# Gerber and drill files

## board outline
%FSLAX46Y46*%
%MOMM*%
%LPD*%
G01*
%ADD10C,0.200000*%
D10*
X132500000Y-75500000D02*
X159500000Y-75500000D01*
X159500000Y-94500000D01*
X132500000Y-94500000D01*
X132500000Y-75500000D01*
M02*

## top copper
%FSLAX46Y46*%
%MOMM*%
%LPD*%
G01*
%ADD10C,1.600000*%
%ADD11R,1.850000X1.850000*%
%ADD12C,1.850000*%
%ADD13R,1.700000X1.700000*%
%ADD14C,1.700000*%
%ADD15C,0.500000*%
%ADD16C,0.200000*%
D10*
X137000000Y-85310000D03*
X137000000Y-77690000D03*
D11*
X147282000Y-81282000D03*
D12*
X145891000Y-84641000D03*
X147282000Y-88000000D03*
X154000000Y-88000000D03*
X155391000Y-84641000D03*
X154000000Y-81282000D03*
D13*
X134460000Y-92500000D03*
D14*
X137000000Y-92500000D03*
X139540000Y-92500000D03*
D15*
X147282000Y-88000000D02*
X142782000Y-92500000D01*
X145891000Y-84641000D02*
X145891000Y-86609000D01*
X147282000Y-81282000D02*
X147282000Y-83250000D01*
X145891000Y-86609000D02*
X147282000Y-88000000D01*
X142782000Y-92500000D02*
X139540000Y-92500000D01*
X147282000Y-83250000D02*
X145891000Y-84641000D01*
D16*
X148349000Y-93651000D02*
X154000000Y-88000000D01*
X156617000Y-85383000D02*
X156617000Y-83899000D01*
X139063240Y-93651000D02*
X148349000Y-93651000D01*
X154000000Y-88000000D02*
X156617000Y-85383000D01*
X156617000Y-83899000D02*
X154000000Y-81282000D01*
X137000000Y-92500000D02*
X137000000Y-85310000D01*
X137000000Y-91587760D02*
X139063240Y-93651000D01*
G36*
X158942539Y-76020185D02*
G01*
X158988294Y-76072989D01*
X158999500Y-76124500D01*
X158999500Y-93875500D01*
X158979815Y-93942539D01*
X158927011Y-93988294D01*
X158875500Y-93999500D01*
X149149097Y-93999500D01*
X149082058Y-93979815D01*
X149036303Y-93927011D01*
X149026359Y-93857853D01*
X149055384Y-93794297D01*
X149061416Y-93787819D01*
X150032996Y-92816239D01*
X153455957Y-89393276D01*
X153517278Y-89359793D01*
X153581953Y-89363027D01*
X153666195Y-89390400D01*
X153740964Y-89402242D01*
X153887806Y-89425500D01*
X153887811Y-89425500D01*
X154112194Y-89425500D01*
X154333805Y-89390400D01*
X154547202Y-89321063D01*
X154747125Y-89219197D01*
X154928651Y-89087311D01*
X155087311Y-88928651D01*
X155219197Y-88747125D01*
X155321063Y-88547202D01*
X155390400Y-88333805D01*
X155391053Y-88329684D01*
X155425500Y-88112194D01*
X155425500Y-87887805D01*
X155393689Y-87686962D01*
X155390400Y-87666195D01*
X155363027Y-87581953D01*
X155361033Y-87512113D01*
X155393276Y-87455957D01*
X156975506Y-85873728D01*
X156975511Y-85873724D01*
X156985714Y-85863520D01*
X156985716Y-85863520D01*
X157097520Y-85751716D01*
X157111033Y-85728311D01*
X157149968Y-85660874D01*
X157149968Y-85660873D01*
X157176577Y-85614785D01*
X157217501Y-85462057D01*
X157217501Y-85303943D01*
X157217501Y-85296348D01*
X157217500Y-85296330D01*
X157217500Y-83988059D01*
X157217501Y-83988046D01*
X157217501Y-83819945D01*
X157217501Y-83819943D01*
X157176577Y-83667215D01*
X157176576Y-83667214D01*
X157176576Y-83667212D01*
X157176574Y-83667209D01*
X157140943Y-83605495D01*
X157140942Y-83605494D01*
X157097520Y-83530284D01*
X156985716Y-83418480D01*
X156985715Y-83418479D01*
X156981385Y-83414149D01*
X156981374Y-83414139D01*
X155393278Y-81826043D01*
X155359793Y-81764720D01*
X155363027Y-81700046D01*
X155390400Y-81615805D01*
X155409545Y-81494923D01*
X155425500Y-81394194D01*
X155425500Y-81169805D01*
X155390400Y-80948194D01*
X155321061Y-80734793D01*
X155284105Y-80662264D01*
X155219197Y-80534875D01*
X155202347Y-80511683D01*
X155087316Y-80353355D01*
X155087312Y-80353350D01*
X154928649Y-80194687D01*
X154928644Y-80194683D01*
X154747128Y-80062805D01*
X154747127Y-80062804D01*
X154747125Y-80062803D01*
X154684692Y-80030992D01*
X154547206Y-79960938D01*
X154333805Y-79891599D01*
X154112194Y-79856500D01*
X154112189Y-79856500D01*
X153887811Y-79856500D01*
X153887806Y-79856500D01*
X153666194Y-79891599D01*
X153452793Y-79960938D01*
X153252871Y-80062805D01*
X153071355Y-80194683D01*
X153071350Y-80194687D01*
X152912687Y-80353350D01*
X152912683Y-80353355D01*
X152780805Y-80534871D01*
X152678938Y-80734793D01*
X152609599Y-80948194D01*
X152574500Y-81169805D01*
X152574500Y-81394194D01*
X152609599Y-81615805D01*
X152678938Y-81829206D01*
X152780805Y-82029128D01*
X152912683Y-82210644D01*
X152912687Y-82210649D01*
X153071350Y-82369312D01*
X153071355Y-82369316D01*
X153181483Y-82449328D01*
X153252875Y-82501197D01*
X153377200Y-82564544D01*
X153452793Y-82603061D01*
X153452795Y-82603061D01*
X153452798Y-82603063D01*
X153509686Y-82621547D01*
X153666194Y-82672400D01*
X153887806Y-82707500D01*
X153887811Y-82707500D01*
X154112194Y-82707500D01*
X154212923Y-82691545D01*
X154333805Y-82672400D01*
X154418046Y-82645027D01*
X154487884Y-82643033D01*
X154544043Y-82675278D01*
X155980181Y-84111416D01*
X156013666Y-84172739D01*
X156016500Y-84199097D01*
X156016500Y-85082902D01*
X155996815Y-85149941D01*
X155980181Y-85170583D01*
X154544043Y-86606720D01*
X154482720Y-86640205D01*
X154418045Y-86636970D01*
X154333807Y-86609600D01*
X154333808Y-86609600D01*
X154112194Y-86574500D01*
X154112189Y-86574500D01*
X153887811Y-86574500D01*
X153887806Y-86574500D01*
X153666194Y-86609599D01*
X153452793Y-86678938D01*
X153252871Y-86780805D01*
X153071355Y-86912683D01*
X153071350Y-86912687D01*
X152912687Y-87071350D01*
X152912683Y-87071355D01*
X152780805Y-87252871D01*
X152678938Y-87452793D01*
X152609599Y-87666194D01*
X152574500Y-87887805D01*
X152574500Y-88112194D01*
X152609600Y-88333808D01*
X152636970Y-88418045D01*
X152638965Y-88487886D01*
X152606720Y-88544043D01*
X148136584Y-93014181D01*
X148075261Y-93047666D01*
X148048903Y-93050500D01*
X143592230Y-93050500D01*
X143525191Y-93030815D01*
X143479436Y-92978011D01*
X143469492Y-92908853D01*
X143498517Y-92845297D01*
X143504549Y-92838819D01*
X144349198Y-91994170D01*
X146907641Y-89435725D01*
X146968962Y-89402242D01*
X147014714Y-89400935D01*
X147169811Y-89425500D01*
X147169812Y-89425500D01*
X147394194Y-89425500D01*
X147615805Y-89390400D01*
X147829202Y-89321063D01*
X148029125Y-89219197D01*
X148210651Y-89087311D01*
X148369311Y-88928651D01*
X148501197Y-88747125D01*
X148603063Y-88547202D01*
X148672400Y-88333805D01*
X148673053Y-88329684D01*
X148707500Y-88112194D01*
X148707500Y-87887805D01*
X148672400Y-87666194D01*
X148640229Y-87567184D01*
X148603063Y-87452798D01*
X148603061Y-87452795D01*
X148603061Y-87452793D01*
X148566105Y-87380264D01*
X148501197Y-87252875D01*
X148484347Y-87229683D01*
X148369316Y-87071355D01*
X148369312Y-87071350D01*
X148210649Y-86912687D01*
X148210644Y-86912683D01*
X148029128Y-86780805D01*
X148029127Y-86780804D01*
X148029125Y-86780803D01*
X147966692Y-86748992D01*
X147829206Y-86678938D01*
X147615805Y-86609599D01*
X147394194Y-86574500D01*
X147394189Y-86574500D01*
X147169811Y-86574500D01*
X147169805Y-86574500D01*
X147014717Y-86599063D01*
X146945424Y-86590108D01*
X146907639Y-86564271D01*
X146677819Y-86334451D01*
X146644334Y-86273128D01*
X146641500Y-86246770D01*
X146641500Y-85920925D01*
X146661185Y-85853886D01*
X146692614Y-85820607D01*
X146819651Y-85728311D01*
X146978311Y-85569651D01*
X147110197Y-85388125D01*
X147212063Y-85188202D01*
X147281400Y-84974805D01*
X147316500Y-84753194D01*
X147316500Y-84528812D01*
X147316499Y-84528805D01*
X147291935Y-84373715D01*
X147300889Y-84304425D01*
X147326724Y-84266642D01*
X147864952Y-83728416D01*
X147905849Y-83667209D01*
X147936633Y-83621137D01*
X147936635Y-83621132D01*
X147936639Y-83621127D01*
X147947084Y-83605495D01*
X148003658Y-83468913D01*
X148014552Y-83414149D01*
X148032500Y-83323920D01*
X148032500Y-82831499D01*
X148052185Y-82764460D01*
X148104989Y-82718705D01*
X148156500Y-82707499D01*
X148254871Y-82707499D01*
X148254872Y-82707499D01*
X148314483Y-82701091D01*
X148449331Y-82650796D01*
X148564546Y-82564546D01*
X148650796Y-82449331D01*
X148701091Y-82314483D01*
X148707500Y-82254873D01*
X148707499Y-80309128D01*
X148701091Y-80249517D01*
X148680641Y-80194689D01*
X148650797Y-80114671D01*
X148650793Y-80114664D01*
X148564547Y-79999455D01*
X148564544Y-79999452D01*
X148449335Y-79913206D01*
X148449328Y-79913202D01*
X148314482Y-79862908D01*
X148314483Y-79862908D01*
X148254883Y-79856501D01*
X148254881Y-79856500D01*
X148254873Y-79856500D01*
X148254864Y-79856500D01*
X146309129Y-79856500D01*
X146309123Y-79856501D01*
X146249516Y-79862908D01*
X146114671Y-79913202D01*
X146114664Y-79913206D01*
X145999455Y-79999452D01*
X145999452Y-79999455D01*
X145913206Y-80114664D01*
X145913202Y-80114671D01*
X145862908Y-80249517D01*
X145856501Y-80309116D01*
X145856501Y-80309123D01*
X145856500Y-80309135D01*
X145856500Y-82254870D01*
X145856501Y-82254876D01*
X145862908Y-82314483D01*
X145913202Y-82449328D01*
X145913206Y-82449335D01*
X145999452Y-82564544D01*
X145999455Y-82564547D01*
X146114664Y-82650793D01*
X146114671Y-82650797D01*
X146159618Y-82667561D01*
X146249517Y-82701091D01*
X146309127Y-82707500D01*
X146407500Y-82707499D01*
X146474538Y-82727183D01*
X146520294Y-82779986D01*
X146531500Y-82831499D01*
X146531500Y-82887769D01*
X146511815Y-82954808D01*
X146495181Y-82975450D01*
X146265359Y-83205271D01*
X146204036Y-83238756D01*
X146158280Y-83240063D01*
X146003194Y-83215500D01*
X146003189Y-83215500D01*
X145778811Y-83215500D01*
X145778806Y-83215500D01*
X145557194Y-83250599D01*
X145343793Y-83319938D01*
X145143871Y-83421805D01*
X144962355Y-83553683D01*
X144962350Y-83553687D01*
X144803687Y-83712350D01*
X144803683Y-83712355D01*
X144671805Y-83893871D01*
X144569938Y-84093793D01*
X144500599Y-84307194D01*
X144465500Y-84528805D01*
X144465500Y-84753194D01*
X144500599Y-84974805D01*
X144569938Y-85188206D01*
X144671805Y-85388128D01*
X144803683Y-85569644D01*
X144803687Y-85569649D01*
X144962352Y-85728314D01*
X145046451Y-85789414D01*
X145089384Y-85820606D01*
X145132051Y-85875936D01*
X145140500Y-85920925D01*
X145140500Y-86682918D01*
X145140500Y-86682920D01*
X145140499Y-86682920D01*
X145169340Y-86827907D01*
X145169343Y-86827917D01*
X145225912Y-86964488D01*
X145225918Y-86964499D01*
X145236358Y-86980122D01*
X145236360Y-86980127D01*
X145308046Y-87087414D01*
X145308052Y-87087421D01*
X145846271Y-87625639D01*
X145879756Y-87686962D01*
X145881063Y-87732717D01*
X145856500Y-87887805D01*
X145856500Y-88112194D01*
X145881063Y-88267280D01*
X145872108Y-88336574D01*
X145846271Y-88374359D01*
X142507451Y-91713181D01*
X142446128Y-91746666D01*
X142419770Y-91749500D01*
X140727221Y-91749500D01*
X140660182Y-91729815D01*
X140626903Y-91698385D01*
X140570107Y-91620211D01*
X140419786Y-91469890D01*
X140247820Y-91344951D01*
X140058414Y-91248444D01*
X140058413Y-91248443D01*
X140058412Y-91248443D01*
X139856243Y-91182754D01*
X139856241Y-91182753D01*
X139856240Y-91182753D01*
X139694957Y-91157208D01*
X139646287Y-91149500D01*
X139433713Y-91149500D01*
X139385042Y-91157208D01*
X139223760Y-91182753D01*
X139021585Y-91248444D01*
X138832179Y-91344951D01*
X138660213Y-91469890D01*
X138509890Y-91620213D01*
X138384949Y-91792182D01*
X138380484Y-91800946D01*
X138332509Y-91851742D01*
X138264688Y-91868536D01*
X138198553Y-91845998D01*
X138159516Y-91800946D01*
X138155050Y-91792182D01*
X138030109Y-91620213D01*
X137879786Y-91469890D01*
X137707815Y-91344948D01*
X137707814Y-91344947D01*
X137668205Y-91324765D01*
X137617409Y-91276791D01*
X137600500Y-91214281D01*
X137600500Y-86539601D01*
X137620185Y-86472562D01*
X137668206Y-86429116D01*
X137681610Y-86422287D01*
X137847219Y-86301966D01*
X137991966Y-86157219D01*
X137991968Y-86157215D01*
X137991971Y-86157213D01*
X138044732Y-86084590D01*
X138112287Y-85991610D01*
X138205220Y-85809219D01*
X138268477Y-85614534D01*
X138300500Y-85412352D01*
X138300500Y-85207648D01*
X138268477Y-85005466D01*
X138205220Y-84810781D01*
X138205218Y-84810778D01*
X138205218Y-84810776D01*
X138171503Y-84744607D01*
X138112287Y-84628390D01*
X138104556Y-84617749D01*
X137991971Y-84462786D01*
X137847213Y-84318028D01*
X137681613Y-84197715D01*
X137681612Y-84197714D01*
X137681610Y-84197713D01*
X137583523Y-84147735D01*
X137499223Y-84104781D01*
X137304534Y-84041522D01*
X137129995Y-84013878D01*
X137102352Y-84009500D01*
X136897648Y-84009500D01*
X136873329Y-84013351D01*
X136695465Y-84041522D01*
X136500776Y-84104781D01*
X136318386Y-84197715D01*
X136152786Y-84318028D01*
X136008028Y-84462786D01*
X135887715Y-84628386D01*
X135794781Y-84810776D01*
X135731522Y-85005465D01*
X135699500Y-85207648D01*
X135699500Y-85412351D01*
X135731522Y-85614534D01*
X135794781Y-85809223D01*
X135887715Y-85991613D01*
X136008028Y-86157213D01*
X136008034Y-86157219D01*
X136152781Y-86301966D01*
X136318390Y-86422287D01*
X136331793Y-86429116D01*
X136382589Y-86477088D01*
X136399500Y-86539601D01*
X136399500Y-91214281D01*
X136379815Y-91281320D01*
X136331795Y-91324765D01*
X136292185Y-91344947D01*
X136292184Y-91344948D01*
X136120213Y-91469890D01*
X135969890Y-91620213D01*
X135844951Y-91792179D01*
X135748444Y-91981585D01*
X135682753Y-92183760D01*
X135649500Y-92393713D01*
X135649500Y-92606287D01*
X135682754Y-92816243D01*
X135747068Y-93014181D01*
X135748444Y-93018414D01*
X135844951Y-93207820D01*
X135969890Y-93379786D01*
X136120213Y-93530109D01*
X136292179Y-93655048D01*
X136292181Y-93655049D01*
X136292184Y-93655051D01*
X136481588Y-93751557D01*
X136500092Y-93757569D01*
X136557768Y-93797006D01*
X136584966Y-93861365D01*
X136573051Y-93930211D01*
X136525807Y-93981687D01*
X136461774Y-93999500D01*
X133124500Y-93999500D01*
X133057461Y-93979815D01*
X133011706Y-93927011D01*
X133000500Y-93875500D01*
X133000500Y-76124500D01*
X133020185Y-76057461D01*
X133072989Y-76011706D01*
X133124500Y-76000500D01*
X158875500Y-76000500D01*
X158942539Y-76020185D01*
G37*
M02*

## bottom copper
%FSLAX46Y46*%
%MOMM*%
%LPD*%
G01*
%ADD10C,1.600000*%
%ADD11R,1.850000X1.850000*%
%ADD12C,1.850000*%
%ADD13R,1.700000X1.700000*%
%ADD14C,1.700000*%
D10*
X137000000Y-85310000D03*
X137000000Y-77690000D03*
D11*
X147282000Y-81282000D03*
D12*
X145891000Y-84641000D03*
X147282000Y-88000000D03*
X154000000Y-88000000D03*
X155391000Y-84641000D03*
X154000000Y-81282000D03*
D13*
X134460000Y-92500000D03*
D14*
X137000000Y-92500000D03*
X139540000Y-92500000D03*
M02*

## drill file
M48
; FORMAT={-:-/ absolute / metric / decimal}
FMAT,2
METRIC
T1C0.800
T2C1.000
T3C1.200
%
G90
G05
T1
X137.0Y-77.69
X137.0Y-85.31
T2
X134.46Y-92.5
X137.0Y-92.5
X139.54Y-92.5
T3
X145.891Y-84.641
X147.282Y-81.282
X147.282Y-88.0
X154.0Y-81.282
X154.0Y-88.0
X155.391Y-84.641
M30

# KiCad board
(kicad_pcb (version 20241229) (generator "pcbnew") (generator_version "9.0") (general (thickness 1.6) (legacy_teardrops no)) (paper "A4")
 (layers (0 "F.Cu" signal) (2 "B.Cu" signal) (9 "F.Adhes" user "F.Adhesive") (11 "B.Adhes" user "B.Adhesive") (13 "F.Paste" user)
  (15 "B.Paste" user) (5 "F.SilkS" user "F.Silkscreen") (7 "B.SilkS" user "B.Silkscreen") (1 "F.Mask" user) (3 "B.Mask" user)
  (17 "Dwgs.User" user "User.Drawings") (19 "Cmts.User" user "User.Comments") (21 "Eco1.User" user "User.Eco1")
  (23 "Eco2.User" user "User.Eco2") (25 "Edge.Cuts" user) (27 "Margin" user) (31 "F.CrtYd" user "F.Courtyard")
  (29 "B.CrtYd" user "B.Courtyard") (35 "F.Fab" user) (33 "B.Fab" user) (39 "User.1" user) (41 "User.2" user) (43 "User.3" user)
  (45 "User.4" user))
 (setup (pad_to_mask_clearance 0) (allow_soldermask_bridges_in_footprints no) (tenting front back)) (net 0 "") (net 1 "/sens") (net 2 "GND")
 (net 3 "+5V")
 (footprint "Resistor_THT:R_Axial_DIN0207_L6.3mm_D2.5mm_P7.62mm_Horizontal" (layer "F.Cu") (at 137 85.31 90)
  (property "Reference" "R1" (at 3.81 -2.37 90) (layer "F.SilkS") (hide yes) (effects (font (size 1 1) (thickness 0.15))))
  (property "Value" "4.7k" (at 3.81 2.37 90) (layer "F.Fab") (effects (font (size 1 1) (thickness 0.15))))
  (pad "1" thru_hole circle (at 0 0 90) (size 1.6 1.6) (drill 0.8) (layers "*.Cu" "*.Mask") (remove_unused_layers no) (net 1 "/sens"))
  (pad "2" thru_hole circle (at 7.62 0 90) (size 1.6 1.6) (drill 0.8) (layers "*.Cu" "*.Mask") (remove_unused_layers no) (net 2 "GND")))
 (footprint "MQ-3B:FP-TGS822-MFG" (layer "F.Cu") (at 150.641 84.641)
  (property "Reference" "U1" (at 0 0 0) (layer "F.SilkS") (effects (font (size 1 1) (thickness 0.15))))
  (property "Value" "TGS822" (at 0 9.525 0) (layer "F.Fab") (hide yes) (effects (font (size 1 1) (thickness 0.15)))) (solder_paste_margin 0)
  (pad "1" thru_hole rect (at -3.359 -3.359) (size 1.85 1.85) (drill 1.2) (layers "*.Cu" "*.Mask") (remove_unused_layers no) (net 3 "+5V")
   (solder_mask_margin 0) (solder_paste_margin -2147.48364))
  (pad "2" thru_hole circle (at -4.75 0) (size 1.85 1.85) (drill 1.2) (layers "*.Cu" "*.Mask") (remove_unused_layers no) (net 3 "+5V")
   (solder_mask_margin 0) (solder_paste_margin -2147.48364) (thermal_bridge_angle 90))
  (pad "3" thru_hole circle (at -3.359 3.359) (size 1.85 1.85) (drill 1.2) (layers "*.Cu" "*.Mask") (remove_unused_layers no) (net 3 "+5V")
   (solder_mask_margin 0) (solder_paste_margin -2147.48364) (thermal_bridge_angle 90))
  (pad "4" thru_hole circle (at 3.359 3.359) (size 1.85 1.85) (drill 1.2) (layers "*.Cu" "*.Mask") (remove_unused_layers no) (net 1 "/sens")
   (solder_mask_margin 0) (solder_paste_margin -2147.48364) (thermal_bridge_angle 90))
  (pad "5" thru_hole circle (at 4.75 0) (size 1.85 1.85) (drill 1.2) (layers "*.Cu" "*.Mask") (remove_unused_layers no) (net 2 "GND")
   (solder_mask_margin 0) (solder_paste_margin -2147.48364) (thermal_bridge_angle 90))
  (pad "6" thru_hole circle (at 3.359 -3.359) (size 1.85 1.85) (drill 1.2) (layers "*.Cu" "*.Mask") (remove_unused_layers no)
   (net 1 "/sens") (solder_mask_margin 0) (solder_paste_margin -2147.48364) (thermal_bridge_angle 90)))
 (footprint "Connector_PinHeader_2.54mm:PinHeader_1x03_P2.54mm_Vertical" (layer "F.Cu") (at 134.46 92.5 90)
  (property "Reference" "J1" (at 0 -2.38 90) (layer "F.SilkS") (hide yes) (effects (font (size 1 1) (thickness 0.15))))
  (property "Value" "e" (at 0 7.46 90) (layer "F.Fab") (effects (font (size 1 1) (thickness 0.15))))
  (pad "1" thru_hole rect (at 0 0 90) (size 1.7 1.7) (drill 1) (layers "*.Cu" "*.Mask") (remove_unused_layers no) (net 2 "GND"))
  (pad "2" thru_hole circle (at 0 2.54 90) (size 1.7 1.7) (drill 1) (layers "*.Cu" "*.Mask") (remove_unused_layers no) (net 1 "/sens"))
  (pad "3" thru_hole circle (at 0 5.08 90) (size 1.7 1.7) (drill 1) (layers "*.Cu" "*.Mask") (remove_unused_layers no) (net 3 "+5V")))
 (gr_rect (start 132.5 75.5) (end 159.5 94.5) (stroke (width 0.2) (type solid)) (fill no) (layer "Edge.Cuts"))
 (segment (start 147.282 88) (end 142.782 92.5) (width 0.5) (layer "F.Cu") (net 3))
 (segment (start 145.891 84.641) (end 145.891 86.609) (width 0.5) (layer "F.Cu") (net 3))
 (segment (start 147.282 81.282) (end 147.282 83.25) (width 0.5) (layer "F.Cu") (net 3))
 (segment (start 145.891 86.609) (end 147.282 88) (width 0.5) (layer "F.Cu") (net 3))
 (segment (start 142.782 92.5) (end 139.54 92.5) (width 0.5) (layer "F.Cu") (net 3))
 (segment (start 147.282 83.25) (end 145.891 84.641) (width 0.5) (layer "F.Cu") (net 3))
 (segment (start 148.349 93.651) (end 154 88) (width 0.2) (layer "F.Cu") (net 1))
 (segment (start 156.617 85.383) (end 156.617 83.899) (width 0.2) (layer "F.Cu") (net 1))
 (segment (start 139.06324 93.651) (end 148.349 93.651) (width 0.2) (layer "F.Cu") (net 1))
 (segment (start 154 88) (end 156.617 85.383) (width 0.2) (layer "F.Cu") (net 1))
 (segment (start 156.617 83.899) (end 154 81.282) (width 0.2) (layer "F.Cu") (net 1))
 (segment (start 137 92.5) (end 137 85.31) (width 0.2) (layer "F.Cu") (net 1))
 (segment (start 137 91.58776) (end 139.06324 93.651) (width 0.2) (layer "F.Cu") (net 1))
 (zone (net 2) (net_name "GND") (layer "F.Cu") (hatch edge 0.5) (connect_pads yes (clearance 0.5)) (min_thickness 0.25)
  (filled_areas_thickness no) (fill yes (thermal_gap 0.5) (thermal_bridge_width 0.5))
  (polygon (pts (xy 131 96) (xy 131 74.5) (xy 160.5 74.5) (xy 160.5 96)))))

